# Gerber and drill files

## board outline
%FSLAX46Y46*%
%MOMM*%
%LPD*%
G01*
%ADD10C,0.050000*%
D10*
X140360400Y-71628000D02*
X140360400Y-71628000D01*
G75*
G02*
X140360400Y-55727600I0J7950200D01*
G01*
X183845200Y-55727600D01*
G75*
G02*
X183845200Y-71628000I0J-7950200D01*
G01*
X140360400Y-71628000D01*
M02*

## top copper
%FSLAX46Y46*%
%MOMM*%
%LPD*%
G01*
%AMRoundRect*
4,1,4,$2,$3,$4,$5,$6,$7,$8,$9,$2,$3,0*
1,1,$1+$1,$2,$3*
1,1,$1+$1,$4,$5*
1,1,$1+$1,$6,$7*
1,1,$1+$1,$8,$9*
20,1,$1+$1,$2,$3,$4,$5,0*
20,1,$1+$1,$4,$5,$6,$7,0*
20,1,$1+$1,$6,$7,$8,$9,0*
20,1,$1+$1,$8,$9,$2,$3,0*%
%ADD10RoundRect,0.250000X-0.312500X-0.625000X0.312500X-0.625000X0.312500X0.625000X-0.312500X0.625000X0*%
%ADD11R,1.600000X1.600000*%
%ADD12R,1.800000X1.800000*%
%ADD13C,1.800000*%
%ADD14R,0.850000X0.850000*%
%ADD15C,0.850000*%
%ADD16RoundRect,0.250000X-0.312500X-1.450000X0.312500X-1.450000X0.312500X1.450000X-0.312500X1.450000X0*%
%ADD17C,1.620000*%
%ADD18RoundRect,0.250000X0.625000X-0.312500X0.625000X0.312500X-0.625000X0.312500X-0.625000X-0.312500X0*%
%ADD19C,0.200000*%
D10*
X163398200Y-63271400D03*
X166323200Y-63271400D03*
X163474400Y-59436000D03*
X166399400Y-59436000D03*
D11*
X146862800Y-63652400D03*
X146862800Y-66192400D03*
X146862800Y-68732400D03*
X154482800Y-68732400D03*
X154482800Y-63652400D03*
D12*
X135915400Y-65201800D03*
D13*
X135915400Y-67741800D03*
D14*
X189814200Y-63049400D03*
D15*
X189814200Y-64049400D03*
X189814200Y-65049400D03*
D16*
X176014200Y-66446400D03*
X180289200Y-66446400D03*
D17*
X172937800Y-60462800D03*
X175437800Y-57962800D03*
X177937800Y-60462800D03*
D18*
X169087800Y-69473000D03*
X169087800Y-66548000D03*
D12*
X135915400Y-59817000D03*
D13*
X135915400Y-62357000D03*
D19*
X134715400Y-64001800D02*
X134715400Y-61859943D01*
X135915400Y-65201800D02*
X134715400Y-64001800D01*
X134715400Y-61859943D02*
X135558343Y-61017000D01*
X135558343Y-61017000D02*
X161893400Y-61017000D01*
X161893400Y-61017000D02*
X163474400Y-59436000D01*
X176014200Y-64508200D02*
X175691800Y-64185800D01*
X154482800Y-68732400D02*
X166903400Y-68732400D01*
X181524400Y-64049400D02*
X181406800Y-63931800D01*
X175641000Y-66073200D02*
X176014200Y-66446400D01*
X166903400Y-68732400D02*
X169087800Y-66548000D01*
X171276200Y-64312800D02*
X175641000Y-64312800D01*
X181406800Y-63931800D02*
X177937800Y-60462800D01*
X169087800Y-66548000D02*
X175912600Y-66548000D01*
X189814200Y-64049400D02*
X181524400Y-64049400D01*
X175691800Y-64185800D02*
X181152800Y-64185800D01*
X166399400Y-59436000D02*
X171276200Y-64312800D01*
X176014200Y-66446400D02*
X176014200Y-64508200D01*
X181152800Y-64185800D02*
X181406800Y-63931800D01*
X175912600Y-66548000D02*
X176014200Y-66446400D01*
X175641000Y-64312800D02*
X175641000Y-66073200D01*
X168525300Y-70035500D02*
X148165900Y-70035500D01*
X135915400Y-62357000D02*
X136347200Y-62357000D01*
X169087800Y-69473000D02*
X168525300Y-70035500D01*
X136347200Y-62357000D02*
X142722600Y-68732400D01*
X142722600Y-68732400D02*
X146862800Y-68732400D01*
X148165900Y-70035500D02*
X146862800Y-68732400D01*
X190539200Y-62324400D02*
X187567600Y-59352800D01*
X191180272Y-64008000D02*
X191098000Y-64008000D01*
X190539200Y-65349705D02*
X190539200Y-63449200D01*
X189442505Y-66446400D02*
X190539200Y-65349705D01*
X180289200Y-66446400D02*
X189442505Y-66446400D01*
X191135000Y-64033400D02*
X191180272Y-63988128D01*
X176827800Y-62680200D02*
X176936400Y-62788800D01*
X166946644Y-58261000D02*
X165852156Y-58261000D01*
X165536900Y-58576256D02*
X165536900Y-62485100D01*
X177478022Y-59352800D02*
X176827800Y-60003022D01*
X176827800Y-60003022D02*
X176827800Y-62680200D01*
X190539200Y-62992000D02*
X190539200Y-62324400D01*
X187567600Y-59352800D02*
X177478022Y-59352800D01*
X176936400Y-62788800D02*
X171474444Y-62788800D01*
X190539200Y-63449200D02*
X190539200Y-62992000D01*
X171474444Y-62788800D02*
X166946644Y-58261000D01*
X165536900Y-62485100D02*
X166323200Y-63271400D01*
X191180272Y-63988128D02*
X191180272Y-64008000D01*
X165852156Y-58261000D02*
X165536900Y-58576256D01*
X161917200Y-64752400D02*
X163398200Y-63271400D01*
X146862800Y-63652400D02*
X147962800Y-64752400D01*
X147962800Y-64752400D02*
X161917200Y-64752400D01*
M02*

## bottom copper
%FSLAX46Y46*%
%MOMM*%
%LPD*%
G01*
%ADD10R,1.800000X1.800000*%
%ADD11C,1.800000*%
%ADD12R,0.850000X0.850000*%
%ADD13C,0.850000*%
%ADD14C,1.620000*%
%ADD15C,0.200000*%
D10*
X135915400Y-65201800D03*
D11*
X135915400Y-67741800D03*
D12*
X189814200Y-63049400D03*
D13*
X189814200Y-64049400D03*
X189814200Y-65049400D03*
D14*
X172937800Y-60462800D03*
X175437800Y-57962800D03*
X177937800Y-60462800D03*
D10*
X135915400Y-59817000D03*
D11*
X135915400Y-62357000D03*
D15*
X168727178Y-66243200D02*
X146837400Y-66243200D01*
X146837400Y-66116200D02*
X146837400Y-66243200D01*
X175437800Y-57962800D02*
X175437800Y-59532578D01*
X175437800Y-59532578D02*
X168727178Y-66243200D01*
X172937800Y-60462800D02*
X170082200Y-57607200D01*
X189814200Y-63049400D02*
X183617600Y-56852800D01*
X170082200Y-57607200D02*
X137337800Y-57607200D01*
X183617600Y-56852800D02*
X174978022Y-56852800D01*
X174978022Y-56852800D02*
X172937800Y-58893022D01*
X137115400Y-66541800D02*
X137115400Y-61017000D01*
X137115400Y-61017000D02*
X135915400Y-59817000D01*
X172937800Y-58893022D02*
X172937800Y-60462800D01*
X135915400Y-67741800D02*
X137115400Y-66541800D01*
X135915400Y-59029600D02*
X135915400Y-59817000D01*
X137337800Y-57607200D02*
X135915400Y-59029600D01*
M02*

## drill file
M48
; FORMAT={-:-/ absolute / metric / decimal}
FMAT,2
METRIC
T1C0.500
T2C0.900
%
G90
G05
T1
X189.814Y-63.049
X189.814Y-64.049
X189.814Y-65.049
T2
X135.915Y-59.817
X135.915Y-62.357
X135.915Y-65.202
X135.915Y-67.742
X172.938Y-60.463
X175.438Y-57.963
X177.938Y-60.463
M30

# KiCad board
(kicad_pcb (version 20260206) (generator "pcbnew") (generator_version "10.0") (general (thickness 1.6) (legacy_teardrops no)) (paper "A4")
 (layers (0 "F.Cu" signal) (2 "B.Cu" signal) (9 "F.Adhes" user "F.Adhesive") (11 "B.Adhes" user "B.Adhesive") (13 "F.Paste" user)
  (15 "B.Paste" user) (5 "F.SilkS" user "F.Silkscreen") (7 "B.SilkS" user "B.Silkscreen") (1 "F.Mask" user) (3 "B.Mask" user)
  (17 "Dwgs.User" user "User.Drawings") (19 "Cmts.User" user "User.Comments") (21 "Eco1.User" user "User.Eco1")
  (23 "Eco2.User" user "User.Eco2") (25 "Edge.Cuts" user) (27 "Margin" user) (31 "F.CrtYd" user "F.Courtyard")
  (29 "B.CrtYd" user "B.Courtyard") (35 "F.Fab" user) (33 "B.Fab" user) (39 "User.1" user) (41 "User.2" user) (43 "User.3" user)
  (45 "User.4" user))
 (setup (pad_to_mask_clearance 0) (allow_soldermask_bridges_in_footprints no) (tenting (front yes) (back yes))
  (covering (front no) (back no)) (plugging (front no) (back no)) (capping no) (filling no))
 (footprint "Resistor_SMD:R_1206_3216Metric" (layer "F.Cu") (at 164.8607 63.2714)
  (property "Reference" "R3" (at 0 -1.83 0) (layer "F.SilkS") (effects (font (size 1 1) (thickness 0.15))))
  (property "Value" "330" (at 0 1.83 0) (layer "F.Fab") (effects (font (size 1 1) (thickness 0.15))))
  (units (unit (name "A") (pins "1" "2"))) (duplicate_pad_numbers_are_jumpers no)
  (pad "1" smd roundrect (at -1.4625 0) (size 1.125 1.75) (layers "F.Cu" "F.Mask" "F.Paste") (roundrect_rratio 0.222222)
   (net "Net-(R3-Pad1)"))
  (pad "2" smd roundrect (at 1.4625 0) (size 1.125 1.75) (layers "F.Cu" "F.Mask" "F.Paste") (roundrect_rratio 0.222222) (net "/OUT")))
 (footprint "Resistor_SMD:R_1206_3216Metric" (layer "F.Cu") (at 164.9369 59.436)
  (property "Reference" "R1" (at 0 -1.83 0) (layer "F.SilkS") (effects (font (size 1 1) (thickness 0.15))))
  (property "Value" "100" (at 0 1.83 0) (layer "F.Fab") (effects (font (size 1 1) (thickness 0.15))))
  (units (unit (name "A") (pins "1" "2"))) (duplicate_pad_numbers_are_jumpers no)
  (pad "1" smd roundrect (at -1.4625 0) (size 1.125 1.75) (layers "F.Cu" "F.Mask" "F.Paste") (roundrect_rratio 0.222222) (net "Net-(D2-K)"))
  (pad "2" smd roundrect (at 1.4625 0) (size 1.125 1.75) (layers "F.Cu" "F.Mask" "F.Paste") (roundrect_rratio 0.222222) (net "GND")))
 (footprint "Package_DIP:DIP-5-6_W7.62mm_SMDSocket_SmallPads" (layer "F.Cu") (at 150.6728 66.1924)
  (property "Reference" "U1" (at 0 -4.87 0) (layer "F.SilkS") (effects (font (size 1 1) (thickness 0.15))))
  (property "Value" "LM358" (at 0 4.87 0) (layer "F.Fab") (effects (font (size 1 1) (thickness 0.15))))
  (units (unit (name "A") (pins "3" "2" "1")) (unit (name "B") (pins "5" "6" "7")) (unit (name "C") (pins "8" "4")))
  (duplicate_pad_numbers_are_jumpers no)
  (pad "1" smd rect (at -3.81 -2.54) (size 1.6 1.6) (layers "F.Cu" "F.Mask" "F.Paste") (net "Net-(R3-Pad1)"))
  (pad "2" smd rect (at -3.81 0) (size 1.6 1.6) (layers "F.Cu" "F.Mask" "F.Paste") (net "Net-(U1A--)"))
  (pad "3" smd rect (at -3.81 2.54) (size 1.6 1.6) (layers "F.Cu" "F.Mask" "F.Paste") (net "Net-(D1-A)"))
  (pad "4" smd rect (at 3.81 2.54) (size 1.6 1.6) (layers "F.Cu" "F.Mask" "F.Paste") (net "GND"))
  (pad "6" smd rect (at 3.81 -2.54) (size 1.6 1.6) (layers "F.Cu" "F.Mask" "F.Paste")))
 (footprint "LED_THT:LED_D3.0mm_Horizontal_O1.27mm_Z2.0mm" (layer "F.Cu") (at 135.9154 65.2018 -90)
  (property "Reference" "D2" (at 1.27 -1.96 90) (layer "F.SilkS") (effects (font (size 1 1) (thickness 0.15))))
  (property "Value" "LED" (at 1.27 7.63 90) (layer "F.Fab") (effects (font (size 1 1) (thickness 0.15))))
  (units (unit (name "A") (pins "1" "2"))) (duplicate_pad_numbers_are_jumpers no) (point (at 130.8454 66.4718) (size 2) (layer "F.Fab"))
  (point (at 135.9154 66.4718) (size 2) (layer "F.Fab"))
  (pad "1" thru_hole rect (at 0 0 270) (size 1.8 1.8) (drill 0.9) (layers "*.Cu" "*.Mask") (remove_unused_layers no) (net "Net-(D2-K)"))
  (pad "2" thru_hole circle (at 2.54 0 270) (size 1.8 1.8) (drill 0.9) (layers "*.Cu" "*.Mask") (remove_unused_layers no) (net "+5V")))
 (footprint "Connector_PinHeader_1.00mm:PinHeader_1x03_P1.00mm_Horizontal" (layer "F.Cu") (at 189.8142 63.0494)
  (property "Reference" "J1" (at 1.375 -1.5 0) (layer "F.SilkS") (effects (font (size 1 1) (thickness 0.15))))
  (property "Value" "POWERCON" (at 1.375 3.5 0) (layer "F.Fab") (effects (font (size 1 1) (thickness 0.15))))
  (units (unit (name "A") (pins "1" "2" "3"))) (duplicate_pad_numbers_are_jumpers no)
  (pad "1" thru_hole rect (at 0 0) (size 0.85 0.85) (drill 0.5) (layers "*.Cu" "*.Mask") (remove_unused_layers no) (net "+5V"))
  (pad "2" thru_hole circle (at 0 1) (size 0.85 0.85) (drill 0.5) (layers "*.Cu" "*.Mask") (remove_unused_layers no) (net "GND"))
  (pad "3" thru_hole circle (at 0 2) (size 0.85 0.85) (drill 0.5) (layers "*.Cu" "*.Mask") (remove_unused_layers no) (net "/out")))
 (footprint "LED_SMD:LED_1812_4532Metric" (layer "F.Cu") (at 178.1517 66.4464)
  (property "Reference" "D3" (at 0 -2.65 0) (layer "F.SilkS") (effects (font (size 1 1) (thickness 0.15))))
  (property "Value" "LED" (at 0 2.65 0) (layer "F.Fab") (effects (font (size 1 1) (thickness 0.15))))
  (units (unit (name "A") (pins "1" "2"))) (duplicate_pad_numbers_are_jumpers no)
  (pad "1" smd roundrect (at -2.1375 0) (size 1.125 3.4) (layers "F.Cu" "F.Mask" "F.Paste") (roundrect_rratio 0.222222) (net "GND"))
  (pad "2" smd roundrect (at 2.1375 0) (size 1.125 3.4) (layers "F.Cu" "F.Mask" "F.Paste") (roundrect_rratio 0.222222) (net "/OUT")))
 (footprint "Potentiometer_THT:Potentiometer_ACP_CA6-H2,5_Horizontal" (layer "F.Cu") (at 172.9378 60.4628 90)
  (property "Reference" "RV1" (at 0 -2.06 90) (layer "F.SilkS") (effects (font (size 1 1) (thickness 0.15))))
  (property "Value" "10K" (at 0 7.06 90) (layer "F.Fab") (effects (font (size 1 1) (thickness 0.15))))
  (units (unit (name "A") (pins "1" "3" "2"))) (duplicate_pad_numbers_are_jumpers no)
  (pad "1" thru_hole circle (at 0 0 90) (size 1.62 1.62) (drill 0.9) (layers "*.Cu" "*.Mask") (remove_unused_layers no) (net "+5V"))
  (pad "2" thru_hole circle (at 2.5 2.5 90) (size 1.62 1.62) (drill 0.9) (layers "*.Cu" "*.Mask") (remove_unused_layers no)
   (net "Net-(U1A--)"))
  (pad "3" thru_hole circle (at 0 5 90) (size 1.62 1.62) (drill 0.9) (layers "*.Cu" "*.Mask") (remove_unused_layers no) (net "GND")))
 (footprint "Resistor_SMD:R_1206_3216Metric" (layer "F.Cu") (at 169.0878 68.0105 90)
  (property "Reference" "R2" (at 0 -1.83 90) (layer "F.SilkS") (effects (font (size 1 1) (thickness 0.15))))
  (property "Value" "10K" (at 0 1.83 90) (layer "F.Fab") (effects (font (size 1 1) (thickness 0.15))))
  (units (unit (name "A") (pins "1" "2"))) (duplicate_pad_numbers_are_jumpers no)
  (pad "1" smd roundrect (at -1.4625 0 90) (size 1.125 1.75) (layers "F.Cu" "F.Mask" "F.Paste") (roundrect_rratio 0.222222)
   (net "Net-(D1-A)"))
  (pad "2" smd roundrect (at 1.4625 0 90) (size 1.125 1.75) (layers "F.Cu" "F.Mask" "F.Paste") (roundrect_rratio 0.222222) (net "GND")))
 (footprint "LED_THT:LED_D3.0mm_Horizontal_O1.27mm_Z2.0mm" (layer "F.Cu") (at 135.9154 59.817 -90)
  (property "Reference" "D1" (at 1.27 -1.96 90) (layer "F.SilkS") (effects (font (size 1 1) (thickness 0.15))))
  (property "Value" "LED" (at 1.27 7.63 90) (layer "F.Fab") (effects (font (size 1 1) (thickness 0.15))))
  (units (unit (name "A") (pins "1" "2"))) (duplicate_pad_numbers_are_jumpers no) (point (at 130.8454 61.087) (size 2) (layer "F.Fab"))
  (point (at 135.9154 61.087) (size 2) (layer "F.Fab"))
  (pad "1" thru_hole rect (at 0 0 270) (size 1.8 1.8) (drill 0.9) (layers "*.Cu" "*.Mask") (remove_unused_layers no) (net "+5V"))
  (pad "2" thru_hole circle (at 2.54 0 270) (size 1.8 1.8) (drill 0.9) (layers "*.Cu" "*.Mask") (remove_unused_layers no) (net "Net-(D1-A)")))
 (gr_rect (start 132.4102 55.7276) (end 191.7954 71.628) (radius 20.8534) (stroke (width 0.05) (type solid)) (fill no) (layer "Edge.Cuts"))
 (segment (start 134.7154 64.0018) (end 134.7154 61.859943) (width 0.2) (layer "F.Cu") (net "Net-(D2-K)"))
 (segment (start 135.9154 65.2018) (end 134.7154 64.0018) (width 0.2) (layer "F.Cu") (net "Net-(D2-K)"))
 (segment (start 134.7154 61.859943) (end 135.558343 61.017) (width 0.2) (layer "F.Cu") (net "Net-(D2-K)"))
 (segment (start 135.558343 61.017) (end 161.8934 61.017) (width 0.2) (layer "F.Cu") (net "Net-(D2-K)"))
 (segment (start 161.8934 61.017) (end 163.4744 59.436) (width 0.2) (layer "F.Cu") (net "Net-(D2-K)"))
 (segment (start 176.0142 64.5082) (end 175.6918 64.1858) (width 0.2) (layer "F.Cu") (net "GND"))
 (segment (start 154.4828 68.7324) (end 166.9034 68.7324) (width 0.2) (layer "F.Cu") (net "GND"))
 (segment (start 181.5244 64.0494) (end 181.4068 63.9318) (width 0.2) (layer "F.Cu") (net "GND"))
 (segment (start 175.641 66.0732) (end 176.0142 66.4464) (width 0.2) (layer "F.Cu") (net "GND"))
 (segment (start 166.9034 68.7324) (end 169.0878 66.548) (width 0.2) (layer "F.Cu") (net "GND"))
 (segment (start 171.2762 64.3128) (end 175.641 64.3128) (width 0.2) (layer "F.Cu") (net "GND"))
 (segment (start 181.4068 63.9318) (end 177.9378 60.4628) (width 0.2) (layer "F.Cu") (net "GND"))
 (segment (start 169.0878 66.548) (end 175.9126 66.548) (width 0.2) (layer "F.Cu") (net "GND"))
 (segment (start 189.8142 64.0494) (end 181.5244 64.0494) (width 0.2) (layer "F.Cu") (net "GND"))
 (segment (start 175.6918 64.1858) (end 181.1528 64.1858) (width 0.2) (layer "F.Cu") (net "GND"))
 (segment (start 166.3994 59.436) (end 171.2762 64.3128) (width 0.2) (layer "F.Cu") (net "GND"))
 (segment (start 176.0142 66.4464) (end 176.0142 64.5082) (width 0.2) (layer "F.Cu") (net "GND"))
 (segment (start 181.1528 64.1858) (end 181.4068 63.9318) (width 0.2) (layer "F.Cu") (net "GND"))
 (segment (start 175.9126 66.548) (end 176.0142 66.4464) (width 0.2) (layer "F.Cu") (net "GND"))
 (segment (start 175.641 64.3128) (end 175.641 66.0732) (width 0.2) (layer "F.Cu") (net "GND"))
 (segment (start 168.5253 70.0355) (end 148.1659 70.0355) (width 0.2) (layer "F.Cu") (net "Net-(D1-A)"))
 (segment (start 135.9154 62.357) (end 136.3472 62.357) (width 0.2) (layer "F.Cu") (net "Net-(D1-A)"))
 (segment (start 169.0878 69.473) (end 168.5253 70.0355) (width 0.2) (layer "F.Cu") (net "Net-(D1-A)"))
 (segment (start 136.3472 62.357) (end 142.7226 68.7324) (width 0.2) (layer "F.Cu") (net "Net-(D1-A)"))
 (segment (start 142.7226 68.7324) (end 146.8628 68.7324) (width 0.2) (layer "F.Cu") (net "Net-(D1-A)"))
 (segment (start 148.1659 70.0355) (end 146.8628 68.7324) (width 0.2) (layer "F.Cu") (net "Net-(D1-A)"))
 (segment (start 190.5392 62.3244) (end 187.5676 59.3528) (width 0.2) (layer "F.Cu") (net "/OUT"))
 (segment (start 191.180272 64.008) (end 191.098 64.008) (width 0.2) (layer "F.Cu") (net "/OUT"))
 (segment (start 190.5392 65.349705) (end 190.5392 63.4492) (width 0.2) (layer "F.Cu") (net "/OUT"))
 (segment (start 189.442505 66.4464) (end 190.5392 65.349705) (width 0.2) (layer "F.Cu") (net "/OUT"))
 (segment (start 180.2892 66.4464) (end 189.442505 66.4464) (width 0.2) (layer "F.Cu") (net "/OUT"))
 (segment (start 191.135 64.0334) (end 191.180272 63.988128) (width 0.2) (layer "F.Cu") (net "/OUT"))
 (segment (start 176.8278 62.6802) (end 176.9364 62.7888) (width 0.2) (layer "F.Cu") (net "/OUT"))
 (segment (start 166.946644 58.261) (end 165.852156 58.261) (width 0.2) (layer "F.Cu") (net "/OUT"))
 (segment (start 165.5369 58.576256) (end 165.5369 62.4851) (width 0.2) (layer "F.Cu") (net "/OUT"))
 (segment (start 177.478022 59.3528) (end 176.8278 60.003022) (width 0.2) (layer "F.Cu") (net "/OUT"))
 (segment (start 176.8278 60.003022) (end 176.8278 62.6802) (width 0.2) (layer "F.Cu") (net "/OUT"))
 (segment (start 190.5392 62.992) (end 190.5392 62.3244) (width 0.2) (layer "F.Cu") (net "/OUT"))
 (segment (start 187.5676 59.3528) (end 177.478022 59.3528) (width 0.2) (layer "F.Cu") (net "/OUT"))
 (segment (start 176.9364 62.7888) (end 171.474444 62.7888) (width 0.2) (layer "F.Cu") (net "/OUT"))
 (segment (start 190.5392 63.4492) (end 190.5392 62.992) (width 0.2) (layer "F.Cu") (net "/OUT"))
 (segment (start 171.474444 62.7888) (end 166.946644 58.261) (width 0.2) (layer "F.Cu") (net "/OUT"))
 (segment (start 165.5369 62.4851) (end 166.3232 63.2714) (width 0.2) (layer "F.Cu") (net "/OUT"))
 (segment (start 191.180272 63.988128) (end 191.180272 64.008) (width 0.2) (layer "F.Cu") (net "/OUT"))
 (segment (start 165.852156 58.261) (end 165.5369 58.576256) (width 0.2) (layer "F.Cu") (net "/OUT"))
 (segment (start 161.9172 64.7524) (end 163.3982 63.2714) (width 0.2) (layer "F.Cu") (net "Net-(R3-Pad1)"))
 (segment (start 146.8628 63.6524) (end 147.9628 64.7524) (width 0.2) (layer "F.Cu") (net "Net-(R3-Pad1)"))
 (segment (start 147.9628 64.7524) (end 161.9172 64.7524) (width 0.2) (layer "F.Cu") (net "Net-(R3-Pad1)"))
 (segment (start 168.727178 66.2432) (end 146.8374 66.2432) (width 0.2) (layer "B.Cu") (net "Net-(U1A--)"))
 (segment (start 146.8374 66.1162) (end 146.8374 66.2432) (width 0.2) (layer "B.Cu") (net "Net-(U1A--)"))
 (segment (start 175.4378 57.9628) (end 175.4378 59.532578) (width 0.2) (layer "B.Cu") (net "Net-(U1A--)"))
 (segment (start 175.4378 59.532578) (end 168.727178 66.2432) (width 0.2) (layer "B.Cu") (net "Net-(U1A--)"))
 (segment (start 172.9378 60.4628) (end 170.0822 57.6072) (width 0.2) (layer "B.Cu") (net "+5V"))
 (segment (start 189.8142 63.0494) (end 183.6176 56.8528) (width 0.2) (layer "B.Cu") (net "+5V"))
 (segment (start 170.0822 57.6072) (end 137.3378 57.6072) (width 0.2) (layer "B.Cu") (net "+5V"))
 (segment (start 183.6176 56.8528) (end 174.978022 56.8528) (width 0.2) (layer "B.Cu") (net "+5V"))
 (segment (start 174.978022 56.8528) (end 172.9378 58.893022) (width 0.2) (layer "B.Cu") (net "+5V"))
 (segment (start 137.1154 66.5418) (end 137.1154 61.017) (width 0.2) (layer "B.Cu") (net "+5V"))
 (segment (start 137.1154 61.017) (end 135.9154 59.817) (width 0.2) (layer "B.Cu") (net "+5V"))
 (segment (start 172.9378 58.893022) (end 172.9378 60.4628) (width 0.2) (layer "B.Cu") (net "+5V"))
 (segment (start 135.9154 67.7418) (end 137.1154 66.5418) (width 0.2) (layer "B.Cu") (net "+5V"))
 (segment (start 135.9154 59.0296) (end 135.9154 59.817) (width 0.2) (layer "B.Cu") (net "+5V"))
 (segment (start 137.3378 57.6072) (end 135.9154 59.0296) (width 0.2) (layer "B.Cu") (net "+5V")))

